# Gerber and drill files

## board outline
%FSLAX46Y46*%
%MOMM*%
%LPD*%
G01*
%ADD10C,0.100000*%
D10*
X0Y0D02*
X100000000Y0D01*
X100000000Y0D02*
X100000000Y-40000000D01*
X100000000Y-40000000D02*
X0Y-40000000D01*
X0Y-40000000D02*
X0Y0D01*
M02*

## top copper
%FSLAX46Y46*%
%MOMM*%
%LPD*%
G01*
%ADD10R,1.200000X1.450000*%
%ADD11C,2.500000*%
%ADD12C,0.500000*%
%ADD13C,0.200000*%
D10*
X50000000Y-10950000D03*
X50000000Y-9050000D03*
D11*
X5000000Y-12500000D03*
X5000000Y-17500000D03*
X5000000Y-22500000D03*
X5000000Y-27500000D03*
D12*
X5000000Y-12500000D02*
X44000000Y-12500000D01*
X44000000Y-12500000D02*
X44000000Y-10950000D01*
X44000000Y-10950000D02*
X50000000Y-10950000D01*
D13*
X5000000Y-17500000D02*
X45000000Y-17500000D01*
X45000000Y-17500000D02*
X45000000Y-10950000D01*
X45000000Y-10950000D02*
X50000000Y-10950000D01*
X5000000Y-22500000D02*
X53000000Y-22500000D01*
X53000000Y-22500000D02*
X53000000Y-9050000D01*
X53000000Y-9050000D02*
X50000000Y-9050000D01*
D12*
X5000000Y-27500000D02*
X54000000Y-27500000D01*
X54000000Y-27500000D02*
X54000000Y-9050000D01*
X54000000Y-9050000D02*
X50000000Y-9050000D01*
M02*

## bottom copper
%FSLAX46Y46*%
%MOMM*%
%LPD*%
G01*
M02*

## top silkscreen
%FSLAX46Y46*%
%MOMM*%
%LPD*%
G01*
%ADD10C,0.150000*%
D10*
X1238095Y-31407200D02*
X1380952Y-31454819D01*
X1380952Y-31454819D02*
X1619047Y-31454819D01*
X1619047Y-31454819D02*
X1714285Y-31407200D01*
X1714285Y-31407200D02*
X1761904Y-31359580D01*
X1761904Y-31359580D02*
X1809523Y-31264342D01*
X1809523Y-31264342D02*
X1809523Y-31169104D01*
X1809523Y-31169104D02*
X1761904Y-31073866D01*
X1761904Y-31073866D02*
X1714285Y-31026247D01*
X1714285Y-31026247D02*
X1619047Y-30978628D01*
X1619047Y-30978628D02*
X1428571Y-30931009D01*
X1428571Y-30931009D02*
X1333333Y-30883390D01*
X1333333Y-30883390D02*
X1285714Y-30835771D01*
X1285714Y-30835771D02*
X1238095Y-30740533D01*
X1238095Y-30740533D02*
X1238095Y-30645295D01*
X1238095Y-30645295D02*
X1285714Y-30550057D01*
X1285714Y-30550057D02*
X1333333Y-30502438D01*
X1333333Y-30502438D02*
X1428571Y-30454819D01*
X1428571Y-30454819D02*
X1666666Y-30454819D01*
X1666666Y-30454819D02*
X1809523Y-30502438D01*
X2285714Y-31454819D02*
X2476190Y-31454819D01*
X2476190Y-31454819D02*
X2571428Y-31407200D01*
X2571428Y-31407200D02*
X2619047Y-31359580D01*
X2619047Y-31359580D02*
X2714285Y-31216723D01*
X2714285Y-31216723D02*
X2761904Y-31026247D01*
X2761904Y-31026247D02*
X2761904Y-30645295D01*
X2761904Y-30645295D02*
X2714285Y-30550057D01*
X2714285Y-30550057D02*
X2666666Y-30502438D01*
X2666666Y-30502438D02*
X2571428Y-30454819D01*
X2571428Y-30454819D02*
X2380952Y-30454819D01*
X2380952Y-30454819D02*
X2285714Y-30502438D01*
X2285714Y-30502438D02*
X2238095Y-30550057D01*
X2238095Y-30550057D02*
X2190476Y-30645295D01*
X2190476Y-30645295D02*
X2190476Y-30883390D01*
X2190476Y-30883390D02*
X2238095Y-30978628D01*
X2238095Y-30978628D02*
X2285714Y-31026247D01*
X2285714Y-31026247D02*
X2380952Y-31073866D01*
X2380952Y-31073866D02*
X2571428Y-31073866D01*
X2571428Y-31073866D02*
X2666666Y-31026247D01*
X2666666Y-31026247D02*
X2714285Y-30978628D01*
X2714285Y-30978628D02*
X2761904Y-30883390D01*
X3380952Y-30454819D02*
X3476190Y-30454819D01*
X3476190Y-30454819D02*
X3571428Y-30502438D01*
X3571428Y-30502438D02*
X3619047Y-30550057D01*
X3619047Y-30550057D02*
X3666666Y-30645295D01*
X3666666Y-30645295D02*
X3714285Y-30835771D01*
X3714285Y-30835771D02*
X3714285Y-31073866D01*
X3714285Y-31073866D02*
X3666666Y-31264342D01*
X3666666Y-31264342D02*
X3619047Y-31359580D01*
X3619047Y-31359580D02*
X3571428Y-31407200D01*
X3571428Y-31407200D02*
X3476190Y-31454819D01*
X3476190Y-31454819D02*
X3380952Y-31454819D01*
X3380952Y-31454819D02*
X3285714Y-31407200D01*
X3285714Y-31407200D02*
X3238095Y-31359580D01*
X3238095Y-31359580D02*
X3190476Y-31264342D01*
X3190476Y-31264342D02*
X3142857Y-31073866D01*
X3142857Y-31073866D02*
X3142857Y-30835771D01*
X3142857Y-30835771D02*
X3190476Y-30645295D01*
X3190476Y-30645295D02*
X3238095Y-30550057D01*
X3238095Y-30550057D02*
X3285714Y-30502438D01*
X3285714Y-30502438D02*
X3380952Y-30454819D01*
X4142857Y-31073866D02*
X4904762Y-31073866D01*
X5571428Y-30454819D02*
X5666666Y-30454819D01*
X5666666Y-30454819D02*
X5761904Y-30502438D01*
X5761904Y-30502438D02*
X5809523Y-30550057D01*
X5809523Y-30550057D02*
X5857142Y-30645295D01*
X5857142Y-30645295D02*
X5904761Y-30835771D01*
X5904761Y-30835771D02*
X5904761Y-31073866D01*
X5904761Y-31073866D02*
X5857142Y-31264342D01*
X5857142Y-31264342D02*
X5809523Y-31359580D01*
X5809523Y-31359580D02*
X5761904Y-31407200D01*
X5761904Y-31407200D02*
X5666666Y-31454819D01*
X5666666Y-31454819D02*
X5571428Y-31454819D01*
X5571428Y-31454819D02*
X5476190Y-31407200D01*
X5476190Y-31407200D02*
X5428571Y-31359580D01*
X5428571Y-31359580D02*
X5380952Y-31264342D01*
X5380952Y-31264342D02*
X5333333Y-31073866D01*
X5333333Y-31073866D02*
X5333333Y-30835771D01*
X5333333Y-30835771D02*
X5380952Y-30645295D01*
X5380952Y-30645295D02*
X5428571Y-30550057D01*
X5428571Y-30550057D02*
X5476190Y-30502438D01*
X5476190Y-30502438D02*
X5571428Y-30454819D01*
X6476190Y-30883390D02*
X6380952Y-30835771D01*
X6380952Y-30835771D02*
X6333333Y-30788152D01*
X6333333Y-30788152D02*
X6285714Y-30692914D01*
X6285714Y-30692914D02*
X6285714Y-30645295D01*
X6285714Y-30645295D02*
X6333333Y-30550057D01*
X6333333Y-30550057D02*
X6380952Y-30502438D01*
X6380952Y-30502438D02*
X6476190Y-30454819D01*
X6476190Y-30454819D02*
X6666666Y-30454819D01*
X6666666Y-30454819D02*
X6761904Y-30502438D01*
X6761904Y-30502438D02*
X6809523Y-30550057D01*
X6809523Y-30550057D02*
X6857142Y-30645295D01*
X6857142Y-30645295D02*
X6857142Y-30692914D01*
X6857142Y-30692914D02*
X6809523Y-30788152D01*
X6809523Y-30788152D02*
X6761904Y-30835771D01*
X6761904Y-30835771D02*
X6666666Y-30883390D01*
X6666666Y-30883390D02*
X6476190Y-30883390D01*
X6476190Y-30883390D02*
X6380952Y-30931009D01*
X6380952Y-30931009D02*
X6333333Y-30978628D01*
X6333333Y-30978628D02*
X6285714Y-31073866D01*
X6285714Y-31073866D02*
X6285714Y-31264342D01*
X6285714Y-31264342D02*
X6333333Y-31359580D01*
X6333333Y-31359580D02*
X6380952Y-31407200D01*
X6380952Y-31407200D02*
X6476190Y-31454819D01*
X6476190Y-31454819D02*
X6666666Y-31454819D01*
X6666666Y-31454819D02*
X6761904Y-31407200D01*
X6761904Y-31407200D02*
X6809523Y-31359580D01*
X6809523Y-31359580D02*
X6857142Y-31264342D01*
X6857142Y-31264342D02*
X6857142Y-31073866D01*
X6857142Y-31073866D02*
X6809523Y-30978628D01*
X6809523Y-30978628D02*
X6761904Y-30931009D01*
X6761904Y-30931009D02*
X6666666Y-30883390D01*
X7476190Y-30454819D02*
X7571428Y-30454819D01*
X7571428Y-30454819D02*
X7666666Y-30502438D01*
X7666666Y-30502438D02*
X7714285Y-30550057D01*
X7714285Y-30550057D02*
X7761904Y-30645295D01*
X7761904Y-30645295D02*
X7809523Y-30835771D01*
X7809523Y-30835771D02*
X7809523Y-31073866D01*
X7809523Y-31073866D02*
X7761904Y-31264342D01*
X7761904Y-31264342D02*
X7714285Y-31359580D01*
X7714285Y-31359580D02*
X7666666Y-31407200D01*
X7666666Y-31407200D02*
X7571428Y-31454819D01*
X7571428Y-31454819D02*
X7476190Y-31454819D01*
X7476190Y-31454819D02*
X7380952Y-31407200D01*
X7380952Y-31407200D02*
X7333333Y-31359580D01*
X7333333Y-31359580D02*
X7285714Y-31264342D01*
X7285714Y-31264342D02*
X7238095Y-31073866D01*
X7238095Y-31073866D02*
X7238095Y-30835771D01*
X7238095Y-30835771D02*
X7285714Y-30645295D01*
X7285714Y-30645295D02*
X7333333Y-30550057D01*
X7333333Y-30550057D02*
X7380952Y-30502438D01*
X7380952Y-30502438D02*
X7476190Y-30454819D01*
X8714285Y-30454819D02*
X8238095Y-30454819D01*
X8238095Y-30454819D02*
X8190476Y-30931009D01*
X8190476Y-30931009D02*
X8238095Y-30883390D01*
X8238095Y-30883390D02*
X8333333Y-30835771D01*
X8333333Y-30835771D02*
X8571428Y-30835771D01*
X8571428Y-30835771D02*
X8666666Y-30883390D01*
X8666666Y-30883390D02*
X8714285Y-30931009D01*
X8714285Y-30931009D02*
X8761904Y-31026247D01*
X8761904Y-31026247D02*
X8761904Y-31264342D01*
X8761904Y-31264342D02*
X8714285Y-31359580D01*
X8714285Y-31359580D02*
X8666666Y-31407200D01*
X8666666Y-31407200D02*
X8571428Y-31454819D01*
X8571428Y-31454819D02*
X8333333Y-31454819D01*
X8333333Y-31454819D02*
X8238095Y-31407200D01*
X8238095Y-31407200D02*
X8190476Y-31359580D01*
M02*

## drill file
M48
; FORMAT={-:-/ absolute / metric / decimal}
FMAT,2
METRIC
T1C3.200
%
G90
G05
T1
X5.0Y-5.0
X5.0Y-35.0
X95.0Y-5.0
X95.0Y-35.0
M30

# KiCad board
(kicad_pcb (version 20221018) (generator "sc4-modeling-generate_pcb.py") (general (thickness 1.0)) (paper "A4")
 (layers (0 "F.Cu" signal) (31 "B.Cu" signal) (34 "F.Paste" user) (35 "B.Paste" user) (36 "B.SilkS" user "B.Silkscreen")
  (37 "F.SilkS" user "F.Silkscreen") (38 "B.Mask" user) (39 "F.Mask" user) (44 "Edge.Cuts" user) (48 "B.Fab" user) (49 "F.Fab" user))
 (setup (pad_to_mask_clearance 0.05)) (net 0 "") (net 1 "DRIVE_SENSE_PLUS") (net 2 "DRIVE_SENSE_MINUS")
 (gr_line (start 0.0 0.0) (end 100.0 0.0) (layer "Edge.Cuts") (width 0.1))
 (gr_line (start 100.0 0.0) (end 100.0 40.0) (layer "Edge.Cuts") (width 0.1))
 (gr_line (start 100.0 40.0) (end 0.0 40.0) (layer "Edge.Cuts") (width 0.1))
 (gr_line (start 0.0 40.0) (end 0.0 0.0) (layer "Edge.Cuts") (width 0.1))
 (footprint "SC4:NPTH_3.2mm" (layer "F.Cu") (at 5.0 5.0)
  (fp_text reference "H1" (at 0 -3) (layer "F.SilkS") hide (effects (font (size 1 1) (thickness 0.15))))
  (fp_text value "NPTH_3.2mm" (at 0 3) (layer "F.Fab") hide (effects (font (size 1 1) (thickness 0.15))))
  (pad "1" np_thru_hole circle (at 0 0) (size 3.2 3.2) (drill 3.2) (layers "*.Cu" "*.Mask")))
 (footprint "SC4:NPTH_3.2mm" (layer "F.Cu") (at 95.0 5.0)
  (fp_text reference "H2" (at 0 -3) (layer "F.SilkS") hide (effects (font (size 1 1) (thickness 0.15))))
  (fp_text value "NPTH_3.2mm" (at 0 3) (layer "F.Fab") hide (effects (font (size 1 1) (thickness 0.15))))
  (pad "1" np_thru_hole circle (at 0 0) (size 3.2 3.2) (drill 3.2) (layers "*.Cu" "*.Mask")))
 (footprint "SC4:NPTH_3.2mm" (layer "F.Cu") (at 5.0 35.0)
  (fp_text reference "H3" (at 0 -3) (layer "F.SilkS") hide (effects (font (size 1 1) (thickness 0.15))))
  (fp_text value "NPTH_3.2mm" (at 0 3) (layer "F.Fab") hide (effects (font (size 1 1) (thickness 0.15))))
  (pad "1" np_thru_hole circle (at 0 0) (size 3.2 3.2) (drill 3.2) (layers "*.Cu" "*.Mask")))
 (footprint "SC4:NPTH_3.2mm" (layer "F.Cu") (at 95.0 35.0)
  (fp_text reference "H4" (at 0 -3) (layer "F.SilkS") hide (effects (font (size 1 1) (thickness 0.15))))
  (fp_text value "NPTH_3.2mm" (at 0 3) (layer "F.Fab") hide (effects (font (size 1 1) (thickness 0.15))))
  (pad "1" np_thru_hole circle (at 0 0) (size 3.2 3.2) (drill 3.2) (layers "*.Cu" "*.Mask")))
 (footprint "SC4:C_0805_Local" (layer "F.Cu") (at 50.0 10.0 90)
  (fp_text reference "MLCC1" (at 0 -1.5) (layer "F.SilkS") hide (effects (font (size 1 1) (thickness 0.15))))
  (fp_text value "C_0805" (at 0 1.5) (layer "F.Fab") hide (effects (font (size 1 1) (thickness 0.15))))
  (pad "1" smd rect (at -0.95 0) (size 1.2 1.45) (layers "F.Cu" "F.Paste" "F.Mask") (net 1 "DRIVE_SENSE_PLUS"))
  (pad "2" smd rect (at 0.95 0) (size 1.2 1.45) (layers "F.Cu" "F.Paste" "F.Mask") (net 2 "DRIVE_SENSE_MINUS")))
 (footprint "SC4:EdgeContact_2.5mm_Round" (layer "F.Cu") (at 5.0 12.5)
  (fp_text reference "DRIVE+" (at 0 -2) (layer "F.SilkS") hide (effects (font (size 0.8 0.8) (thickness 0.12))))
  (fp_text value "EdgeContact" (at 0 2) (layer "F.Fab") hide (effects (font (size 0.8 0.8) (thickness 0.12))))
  (pad "1" smd circle (at 0 0) (size 2.5 2.5) (layers "F.Cu" "F.Mask") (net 1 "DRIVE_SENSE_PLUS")))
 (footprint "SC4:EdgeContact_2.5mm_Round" (layer "F.Cu") (at 5.0 17.5)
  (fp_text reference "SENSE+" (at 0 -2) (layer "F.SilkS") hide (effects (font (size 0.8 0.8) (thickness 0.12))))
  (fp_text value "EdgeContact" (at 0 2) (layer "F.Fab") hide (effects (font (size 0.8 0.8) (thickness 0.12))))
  (pad "1" smd circle (at 0 0) (size 2.5 2.5) (layers "F.Cu" "F.Mask") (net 1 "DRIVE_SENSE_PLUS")))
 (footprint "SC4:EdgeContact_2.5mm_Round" (layer "F.Cu") (at 5.0 22.5)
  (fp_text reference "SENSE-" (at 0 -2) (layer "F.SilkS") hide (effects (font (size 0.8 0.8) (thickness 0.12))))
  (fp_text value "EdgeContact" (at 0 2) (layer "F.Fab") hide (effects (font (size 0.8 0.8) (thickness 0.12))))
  (pad "1" smd circle (at 0 0) (size 2.5 2.5) (layers "F.Cu" "F.Mask") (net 2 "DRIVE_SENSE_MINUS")))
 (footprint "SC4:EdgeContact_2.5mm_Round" (layer "F.Cu") (at 5.0 27.5)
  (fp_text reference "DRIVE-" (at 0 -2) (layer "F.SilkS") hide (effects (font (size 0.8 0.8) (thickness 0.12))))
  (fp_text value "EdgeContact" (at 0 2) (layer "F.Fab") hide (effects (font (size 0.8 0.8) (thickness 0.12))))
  (pad "1" smd circle (at 0 0) (size 2.5 2.5) (layers "F.Cu" "F.Mask") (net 2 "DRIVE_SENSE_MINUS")))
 (segment (start 5.0 12.5) (end 44.0 12.5) (width 0.5) (layer "F.Cu") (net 1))
 (segment (start 44.0 12.5) (end 44.0 10.95) (width 0.5) (layer "F.Cu") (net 1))
 (segment (start 44.0 10.95) (end 50.0 10.95) (width 0.5) (layer "F.Cu") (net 1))
 (segment (start 5.0 17.5) (end 45.0 17.5) (width 0.2) (layer "F.Cu") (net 1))
 (segment (start 45.0 17.5) (end 45.0 10.95) (width 0.2) (layer "F.Cu") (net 1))
 (segment (start 45.0 10.95) (end 50.0 10.95) (width 0.2) (layer "F.Cu") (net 1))
 (segment (start 5.0 22.5) (end 53.0 22.5) (width 0.2) (layer "F.Cu") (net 2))
 (segment (start 53.0 22.5) (end 53.0 9.05) (width 0.2) (layer "F.Cu") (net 2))
 (segment (start 53.0 9.05) (end 50.0 9.05) (width 0.2) (layer "F.Cu") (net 2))
 (segment (start 5.0 27.5) (end 54.0 27.5) (width 0.5) (layer "F.Cu") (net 2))
 (segment (start 54.0 27.5) (end 54.0 9.05) (width 0.5) (layer "F.Cu") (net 2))
 (segment (start 54.0 9.05) (end 50.0 9.05) (width 0.5) (layer "F.Cu") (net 2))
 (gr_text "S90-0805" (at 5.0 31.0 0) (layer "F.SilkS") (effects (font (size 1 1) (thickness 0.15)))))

